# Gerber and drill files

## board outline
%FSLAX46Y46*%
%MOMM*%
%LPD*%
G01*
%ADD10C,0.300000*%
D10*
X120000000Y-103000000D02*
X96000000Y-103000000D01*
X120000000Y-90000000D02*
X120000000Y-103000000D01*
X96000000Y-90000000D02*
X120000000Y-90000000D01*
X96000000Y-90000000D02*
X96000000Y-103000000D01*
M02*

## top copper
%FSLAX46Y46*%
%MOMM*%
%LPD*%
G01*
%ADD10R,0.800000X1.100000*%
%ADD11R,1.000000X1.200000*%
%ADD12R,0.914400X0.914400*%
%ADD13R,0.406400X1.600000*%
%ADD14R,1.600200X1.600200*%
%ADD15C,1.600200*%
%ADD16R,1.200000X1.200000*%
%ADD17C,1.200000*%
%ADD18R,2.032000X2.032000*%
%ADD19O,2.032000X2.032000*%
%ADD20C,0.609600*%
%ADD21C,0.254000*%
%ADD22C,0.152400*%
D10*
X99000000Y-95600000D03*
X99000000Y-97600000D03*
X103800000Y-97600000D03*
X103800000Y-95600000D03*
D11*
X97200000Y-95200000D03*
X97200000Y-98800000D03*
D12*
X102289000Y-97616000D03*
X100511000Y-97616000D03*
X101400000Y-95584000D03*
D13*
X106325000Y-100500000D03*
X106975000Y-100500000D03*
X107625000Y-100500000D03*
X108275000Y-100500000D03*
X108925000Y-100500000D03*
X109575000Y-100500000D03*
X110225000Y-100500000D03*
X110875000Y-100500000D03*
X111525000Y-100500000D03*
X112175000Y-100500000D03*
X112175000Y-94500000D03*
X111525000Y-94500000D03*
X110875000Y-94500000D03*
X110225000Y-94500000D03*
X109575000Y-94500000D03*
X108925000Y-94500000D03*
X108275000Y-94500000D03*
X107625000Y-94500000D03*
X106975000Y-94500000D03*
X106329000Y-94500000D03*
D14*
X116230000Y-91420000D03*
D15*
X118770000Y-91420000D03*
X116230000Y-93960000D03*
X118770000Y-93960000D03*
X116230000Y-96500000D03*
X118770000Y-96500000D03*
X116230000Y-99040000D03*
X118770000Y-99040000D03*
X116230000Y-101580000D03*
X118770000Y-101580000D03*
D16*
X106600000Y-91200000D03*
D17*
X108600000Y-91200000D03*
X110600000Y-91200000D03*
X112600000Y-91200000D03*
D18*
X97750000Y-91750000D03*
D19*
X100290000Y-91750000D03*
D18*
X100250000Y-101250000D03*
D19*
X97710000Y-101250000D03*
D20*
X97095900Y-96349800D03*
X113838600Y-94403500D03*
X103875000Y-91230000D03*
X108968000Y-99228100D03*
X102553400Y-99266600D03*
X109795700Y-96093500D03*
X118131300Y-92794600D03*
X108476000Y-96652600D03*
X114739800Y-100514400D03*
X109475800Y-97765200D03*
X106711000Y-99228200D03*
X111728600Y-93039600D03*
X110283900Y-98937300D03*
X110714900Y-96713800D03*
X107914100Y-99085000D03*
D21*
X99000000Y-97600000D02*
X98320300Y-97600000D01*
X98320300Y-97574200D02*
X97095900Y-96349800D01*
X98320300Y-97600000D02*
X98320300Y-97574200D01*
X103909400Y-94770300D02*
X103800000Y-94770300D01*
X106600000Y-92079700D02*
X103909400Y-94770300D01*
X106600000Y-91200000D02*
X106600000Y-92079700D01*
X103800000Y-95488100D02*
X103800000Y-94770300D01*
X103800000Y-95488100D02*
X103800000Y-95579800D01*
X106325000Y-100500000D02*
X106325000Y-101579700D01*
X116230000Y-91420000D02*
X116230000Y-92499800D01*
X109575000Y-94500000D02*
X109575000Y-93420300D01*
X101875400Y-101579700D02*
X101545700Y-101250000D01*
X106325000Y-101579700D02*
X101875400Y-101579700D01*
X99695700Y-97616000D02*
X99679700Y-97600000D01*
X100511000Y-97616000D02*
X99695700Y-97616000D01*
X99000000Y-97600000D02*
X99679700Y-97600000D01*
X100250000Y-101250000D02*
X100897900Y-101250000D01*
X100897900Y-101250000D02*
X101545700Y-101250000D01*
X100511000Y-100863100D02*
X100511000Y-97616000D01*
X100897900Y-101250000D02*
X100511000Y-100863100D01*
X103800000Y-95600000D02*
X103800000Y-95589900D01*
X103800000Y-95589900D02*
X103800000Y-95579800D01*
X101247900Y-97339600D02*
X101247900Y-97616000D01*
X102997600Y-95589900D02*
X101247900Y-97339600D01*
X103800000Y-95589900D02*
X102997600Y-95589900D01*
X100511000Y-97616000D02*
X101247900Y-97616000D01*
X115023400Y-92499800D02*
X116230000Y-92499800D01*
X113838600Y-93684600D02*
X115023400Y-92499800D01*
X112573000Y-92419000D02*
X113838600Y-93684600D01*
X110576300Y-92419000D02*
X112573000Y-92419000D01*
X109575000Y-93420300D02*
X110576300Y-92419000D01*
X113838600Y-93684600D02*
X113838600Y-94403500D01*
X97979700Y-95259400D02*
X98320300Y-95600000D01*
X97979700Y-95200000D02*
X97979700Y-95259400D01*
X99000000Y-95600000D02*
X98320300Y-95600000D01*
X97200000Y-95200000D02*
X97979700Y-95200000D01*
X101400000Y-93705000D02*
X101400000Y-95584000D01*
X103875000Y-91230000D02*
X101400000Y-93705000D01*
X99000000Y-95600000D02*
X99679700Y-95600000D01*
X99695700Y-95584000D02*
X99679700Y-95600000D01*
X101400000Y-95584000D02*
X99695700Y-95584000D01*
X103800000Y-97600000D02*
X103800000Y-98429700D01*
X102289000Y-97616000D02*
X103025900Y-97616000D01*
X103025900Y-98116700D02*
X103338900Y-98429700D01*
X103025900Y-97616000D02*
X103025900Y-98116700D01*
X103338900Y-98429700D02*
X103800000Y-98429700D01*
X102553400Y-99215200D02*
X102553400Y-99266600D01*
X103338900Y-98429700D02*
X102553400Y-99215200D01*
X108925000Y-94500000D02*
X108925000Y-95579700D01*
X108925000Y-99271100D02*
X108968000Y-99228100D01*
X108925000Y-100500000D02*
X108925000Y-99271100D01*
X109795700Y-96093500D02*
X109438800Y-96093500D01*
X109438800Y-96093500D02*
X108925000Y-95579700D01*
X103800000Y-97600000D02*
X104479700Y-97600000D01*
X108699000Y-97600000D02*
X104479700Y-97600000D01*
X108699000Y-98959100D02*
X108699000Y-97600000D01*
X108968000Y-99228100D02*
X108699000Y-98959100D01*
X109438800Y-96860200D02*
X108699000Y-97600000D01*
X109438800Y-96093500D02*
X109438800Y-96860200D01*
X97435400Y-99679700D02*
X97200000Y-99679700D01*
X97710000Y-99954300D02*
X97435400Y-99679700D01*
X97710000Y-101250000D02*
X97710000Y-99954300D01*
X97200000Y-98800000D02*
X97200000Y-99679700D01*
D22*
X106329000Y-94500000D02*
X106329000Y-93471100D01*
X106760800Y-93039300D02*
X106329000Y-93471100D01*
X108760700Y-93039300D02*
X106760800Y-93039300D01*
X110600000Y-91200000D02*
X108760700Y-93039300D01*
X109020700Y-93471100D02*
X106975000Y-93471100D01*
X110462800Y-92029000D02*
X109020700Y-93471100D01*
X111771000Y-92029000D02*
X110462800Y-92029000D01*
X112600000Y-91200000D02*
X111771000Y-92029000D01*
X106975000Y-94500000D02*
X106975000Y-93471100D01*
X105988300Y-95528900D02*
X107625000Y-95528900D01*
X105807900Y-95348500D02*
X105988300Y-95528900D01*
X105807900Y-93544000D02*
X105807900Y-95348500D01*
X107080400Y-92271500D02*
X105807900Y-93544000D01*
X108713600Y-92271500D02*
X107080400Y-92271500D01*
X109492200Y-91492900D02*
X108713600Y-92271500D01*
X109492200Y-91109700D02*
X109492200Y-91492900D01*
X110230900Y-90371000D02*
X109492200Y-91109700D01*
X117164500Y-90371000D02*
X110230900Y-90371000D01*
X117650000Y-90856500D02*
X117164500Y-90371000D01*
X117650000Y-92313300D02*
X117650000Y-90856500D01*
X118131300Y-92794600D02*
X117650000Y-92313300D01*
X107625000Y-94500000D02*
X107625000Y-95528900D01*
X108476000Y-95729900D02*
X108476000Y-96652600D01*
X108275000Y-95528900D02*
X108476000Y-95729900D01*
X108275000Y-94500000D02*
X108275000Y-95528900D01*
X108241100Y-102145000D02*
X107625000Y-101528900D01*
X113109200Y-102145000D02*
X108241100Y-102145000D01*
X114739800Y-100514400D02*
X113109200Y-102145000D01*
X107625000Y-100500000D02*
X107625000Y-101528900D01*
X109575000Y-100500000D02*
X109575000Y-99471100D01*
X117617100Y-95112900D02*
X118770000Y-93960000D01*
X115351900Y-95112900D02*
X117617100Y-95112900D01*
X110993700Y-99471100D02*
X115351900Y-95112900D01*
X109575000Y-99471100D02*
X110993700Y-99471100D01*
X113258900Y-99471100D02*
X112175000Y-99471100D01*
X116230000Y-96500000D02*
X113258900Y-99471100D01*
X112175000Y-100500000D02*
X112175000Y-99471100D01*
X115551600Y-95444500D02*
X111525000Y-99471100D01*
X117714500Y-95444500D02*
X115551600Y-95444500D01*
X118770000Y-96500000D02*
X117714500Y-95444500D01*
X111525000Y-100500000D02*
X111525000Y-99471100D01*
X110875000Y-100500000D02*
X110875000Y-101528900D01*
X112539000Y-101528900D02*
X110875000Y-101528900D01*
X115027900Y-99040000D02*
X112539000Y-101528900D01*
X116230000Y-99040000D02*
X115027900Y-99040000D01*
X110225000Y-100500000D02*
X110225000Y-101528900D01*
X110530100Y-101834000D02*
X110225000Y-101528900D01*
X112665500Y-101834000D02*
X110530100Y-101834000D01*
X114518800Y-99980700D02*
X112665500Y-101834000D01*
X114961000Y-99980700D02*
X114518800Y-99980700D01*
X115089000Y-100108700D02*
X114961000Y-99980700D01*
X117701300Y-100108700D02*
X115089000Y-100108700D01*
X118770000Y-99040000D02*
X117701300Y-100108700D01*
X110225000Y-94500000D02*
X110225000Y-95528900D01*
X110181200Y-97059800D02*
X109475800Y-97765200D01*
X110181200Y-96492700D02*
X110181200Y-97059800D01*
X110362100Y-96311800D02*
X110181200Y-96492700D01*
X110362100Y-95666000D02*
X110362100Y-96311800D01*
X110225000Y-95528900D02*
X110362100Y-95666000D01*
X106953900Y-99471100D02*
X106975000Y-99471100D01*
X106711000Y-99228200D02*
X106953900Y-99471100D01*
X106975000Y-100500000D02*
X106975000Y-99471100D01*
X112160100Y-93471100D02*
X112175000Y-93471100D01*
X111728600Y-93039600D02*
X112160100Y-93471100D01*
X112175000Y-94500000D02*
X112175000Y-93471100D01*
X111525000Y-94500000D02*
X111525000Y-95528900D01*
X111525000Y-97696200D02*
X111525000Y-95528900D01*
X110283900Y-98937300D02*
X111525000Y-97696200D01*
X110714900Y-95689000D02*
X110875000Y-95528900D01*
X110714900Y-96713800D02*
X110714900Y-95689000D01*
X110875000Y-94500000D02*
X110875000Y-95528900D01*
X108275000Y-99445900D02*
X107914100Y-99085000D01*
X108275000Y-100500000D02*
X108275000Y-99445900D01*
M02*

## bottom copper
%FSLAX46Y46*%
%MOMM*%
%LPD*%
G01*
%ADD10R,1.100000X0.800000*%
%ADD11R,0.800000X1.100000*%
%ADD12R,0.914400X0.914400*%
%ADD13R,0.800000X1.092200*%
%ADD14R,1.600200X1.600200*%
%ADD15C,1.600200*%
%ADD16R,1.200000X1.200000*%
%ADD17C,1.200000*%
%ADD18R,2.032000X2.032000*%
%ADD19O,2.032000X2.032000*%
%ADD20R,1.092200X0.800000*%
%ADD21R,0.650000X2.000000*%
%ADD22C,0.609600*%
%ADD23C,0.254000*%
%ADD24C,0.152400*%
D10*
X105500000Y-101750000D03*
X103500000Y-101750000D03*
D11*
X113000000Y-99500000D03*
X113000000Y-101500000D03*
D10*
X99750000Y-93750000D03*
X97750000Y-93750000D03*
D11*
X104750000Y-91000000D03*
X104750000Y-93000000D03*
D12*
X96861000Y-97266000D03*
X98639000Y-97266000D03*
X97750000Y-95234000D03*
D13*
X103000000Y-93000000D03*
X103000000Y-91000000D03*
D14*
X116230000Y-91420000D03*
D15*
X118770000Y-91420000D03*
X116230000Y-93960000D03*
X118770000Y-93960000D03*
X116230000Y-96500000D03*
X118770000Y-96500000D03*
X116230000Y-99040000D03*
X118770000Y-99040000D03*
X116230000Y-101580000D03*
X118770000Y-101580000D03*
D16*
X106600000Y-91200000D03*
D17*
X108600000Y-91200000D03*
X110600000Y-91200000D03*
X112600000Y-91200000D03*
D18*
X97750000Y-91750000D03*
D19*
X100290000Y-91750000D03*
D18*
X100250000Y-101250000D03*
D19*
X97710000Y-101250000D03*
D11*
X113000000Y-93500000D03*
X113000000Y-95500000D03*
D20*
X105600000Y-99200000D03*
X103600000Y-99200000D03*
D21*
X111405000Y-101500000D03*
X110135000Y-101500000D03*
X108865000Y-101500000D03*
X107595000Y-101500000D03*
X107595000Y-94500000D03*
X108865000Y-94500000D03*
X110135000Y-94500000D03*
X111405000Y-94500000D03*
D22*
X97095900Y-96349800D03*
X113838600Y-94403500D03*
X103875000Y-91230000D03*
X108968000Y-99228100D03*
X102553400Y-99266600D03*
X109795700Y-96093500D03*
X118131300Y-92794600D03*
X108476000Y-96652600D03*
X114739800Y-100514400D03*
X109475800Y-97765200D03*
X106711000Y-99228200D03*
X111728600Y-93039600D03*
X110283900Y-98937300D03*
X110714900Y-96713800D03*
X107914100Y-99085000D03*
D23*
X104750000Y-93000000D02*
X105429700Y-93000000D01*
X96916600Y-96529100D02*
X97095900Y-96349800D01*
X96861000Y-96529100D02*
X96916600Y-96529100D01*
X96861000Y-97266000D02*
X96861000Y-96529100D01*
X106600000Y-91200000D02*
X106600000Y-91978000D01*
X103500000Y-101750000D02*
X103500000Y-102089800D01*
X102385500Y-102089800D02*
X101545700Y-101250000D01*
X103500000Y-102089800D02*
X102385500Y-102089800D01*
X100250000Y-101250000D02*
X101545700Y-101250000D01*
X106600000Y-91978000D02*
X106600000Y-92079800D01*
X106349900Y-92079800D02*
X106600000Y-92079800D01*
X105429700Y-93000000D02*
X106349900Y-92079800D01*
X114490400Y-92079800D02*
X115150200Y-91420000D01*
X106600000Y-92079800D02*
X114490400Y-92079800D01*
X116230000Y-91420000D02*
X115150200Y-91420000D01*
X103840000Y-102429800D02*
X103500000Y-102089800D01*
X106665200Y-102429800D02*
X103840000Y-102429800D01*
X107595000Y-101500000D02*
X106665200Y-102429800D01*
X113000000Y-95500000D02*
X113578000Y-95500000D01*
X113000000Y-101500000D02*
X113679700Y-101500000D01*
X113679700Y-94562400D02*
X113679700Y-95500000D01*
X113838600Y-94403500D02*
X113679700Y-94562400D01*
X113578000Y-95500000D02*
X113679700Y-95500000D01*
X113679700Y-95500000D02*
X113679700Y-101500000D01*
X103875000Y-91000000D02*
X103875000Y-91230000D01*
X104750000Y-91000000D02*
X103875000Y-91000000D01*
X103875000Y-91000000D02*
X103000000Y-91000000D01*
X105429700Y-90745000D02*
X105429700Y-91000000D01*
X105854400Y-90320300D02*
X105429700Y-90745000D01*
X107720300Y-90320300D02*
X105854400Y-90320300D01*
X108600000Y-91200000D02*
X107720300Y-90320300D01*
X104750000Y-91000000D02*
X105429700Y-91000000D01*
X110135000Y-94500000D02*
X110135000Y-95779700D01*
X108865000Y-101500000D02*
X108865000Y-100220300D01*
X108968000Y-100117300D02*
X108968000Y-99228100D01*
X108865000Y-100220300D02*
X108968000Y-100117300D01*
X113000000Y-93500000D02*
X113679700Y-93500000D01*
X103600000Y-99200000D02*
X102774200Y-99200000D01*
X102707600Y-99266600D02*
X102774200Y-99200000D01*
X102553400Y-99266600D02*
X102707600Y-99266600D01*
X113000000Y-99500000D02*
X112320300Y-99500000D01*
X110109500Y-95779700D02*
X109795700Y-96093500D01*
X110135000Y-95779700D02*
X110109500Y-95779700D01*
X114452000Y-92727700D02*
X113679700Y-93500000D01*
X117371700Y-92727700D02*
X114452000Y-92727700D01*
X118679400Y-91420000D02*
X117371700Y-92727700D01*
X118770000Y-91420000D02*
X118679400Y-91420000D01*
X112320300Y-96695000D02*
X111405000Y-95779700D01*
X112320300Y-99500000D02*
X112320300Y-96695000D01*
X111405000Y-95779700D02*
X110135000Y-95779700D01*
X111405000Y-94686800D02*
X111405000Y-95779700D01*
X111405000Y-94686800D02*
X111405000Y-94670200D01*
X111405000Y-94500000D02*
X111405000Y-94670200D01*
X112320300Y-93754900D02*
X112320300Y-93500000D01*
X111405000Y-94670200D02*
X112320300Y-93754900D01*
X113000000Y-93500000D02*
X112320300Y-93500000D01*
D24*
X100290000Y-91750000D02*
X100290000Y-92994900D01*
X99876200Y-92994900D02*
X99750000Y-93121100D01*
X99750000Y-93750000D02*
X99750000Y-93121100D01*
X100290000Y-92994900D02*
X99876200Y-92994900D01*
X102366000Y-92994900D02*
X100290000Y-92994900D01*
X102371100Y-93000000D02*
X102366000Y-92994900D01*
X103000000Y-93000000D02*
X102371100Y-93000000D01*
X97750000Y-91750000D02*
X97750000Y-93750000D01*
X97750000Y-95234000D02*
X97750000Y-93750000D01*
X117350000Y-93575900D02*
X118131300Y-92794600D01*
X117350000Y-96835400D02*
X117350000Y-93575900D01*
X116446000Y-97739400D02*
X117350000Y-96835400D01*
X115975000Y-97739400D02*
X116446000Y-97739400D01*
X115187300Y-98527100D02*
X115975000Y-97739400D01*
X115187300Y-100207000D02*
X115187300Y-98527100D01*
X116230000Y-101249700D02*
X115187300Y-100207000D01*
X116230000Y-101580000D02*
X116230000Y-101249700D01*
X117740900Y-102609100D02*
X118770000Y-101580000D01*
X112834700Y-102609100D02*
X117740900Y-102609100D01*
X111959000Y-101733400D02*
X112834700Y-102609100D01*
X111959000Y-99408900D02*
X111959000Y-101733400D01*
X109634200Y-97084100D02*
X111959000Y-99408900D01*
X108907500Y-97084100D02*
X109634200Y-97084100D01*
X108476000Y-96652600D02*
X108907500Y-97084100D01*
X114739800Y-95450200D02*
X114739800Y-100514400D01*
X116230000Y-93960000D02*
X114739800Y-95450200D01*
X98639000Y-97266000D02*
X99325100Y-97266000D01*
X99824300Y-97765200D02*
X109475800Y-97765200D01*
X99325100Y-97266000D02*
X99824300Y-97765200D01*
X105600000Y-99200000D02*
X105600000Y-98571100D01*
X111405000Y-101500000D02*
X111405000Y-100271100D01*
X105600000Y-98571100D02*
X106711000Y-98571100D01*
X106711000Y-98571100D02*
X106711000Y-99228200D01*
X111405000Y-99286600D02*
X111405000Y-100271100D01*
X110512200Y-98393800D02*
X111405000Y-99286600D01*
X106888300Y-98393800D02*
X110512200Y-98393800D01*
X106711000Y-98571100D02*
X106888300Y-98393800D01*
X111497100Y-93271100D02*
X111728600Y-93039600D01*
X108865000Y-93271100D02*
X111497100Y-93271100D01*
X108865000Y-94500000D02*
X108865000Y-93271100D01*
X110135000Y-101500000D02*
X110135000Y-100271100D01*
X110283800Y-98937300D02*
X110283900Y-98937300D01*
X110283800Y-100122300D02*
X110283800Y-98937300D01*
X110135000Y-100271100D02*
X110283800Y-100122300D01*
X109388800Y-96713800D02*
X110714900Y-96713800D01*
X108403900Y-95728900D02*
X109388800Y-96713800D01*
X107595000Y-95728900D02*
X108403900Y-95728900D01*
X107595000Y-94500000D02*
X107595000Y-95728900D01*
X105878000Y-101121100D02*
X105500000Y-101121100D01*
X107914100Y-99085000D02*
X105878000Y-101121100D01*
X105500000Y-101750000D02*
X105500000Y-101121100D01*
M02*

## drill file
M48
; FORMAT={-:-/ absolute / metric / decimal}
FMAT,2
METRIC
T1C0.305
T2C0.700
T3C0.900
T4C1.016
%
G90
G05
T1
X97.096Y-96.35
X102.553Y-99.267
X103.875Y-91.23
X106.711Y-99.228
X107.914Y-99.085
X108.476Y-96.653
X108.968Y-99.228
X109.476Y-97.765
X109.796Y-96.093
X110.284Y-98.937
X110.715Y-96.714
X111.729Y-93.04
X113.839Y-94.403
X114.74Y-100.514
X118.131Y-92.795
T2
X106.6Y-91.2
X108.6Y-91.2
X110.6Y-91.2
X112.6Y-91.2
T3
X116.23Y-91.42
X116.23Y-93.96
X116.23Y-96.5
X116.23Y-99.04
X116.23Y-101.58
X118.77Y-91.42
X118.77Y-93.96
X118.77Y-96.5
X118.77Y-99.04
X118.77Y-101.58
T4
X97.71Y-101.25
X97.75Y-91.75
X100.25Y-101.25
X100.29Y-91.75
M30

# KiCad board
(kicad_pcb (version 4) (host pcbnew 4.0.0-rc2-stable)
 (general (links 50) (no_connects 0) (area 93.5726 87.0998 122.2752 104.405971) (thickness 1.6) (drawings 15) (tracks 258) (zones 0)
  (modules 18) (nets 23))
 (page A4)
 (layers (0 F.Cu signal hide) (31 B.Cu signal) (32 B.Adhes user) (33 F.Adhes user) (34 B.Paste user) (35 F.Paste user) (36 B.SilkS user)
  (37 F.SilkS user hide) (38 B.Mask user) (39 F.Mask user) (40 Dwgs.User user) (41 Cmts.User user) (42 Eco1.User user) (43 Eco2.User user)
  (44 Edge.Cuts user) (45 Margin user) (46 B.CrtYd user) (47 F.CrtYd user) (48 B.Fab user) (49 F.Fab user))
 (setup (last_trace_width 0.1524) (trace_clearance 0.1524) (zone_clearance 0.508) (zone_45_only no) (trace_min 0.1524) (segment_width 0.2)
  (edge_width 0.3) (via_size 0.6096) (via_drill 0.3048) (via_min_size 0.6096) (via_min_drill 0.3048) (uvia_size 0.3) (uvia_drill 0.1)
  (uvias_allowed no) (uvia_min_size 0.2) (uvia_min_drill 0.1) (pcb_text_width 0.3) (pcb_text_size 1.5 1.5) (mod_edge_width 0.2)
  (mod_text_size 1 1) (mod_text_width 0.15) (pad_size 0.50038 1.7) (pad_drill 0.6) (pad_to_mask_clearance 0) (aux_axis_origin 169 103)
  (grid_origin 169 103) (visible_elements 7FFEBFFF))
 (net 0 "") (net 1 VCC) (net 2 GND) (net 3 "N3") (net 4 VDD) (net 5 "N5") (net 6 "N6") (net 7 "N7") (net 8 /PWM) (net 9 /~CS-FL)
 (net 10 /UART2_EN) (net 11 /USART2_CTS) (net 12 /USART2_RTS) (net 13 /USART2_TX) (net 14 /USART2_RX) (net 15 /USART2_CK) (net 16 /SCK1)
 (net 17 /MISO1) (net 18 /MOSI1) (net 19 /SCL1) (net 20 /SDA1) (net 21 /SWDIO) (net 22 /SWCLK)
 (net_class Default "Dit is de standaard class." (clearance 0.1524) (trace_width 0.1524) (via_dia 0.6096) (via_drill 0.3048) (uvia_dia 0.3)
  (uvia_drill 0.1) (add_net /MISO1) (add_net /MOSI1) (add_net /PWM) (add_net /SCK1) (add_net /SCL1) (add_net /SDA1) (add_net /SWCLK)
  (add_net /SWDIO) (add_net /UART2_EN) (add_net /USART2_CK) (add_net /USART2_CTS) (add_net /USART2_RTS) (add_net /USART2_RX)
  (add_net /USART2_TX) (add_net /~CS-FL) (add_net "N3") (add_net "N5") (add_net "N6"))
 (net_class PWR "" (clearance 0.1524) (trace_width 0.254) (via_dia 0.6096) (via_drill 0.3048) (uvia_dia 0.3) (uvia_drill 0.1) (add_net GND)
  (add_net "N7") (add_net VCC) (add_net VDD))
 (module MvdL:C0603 (layer F.Cu) (at 99 96.6 270)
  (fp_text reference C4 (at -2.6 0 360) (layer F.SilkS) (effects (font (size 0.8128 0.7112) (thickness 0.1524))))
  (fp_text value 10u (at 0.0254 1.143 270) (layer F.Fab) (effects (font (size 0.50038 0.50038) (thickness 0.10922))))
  (pad 1 smd rect (at -1 0 270) (size 1.1 0.8) (layers F.Cu F.Paste F.Mask) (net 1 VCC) (clearance 0.1524))
  (pad 2 smd rect (at 1 0 270) (size 1.1 0.8) (layers F.Cu F.Paste F.Mask) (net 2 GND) (clearance 0.1524)))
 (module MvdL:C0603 (layer B.Cu) (at 104.5 101.75 180)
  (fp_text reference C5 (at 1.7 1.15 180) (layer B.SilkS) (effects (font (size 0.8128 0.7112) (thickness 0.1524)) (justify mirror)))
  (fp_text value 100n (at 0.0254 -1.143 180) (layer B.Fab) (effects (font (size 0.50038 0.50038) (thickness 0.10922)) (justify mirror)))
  (pad 1 smd rect (at -1 0 180) (size 1.1 0.8) (layers B.Cu B.Paste B.Mask) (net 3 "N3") (clearance 0.1524))
  (pad 2 smd rect (at 1 0 180) (size 1.1 0.8) (layers B.Cu B.Paste B.Mask) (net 2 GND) (clearance 0.1524)))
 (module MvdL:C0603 (layer F.Cu) (at 103.8 96.6 90)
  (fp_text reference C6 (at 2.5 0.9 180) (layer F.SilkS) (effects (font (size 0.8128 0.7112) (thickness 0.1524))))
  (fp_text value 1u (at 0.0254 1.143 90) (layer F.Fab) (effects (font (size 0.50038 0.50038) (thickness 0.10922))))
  (pad 1 smd rect (at -1 0 90) (size 1.1 0.8) (layers F.Cu F.Paste F.Mask) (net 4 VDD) (clearance 0.1524))
  (pad 2 smd rect (at 1 0 90) (size 1.1 0.8) (layers F.Cu F.Paste F.Mask) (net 2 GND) (clearance 0.1524)))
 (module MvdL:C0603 (layer B.Cu) (at 113 100.5 270)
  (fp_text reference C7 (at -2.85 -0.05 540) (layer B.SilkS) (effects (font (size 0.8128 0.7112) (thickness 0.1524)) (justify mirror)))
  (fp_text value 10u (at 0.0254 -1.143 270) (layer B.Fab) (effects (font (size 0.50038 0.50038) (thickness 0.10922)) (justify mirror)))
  (pad 1 smd rect (at -1 0 270) (size 1.1 0.8) (layers B.Cu B.Paste B.Mask) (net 4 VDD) (clearance 0.1524))
  (pad 2 smd rect (at 1 0 270) (size 1.1 0.8) (layers B.Cu B.Paste B.Mask) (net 2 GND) (clearance 0.1524)))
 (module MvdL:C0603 (layer B.Cu) (at 98.75 93.75 180)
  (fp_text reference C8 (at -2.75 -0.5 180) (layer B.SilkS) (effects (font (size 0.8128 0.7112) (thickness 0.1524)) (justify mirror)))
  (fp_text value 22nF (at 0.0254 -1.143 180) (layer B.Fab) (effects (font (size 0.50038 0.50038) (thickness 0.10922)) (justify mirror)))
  (pad 1 smd rect (at -1 0 180) (size 1.1 0.8) (layers B.Cu B.Paste B.Mask) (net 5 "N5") (clearance 0.1524))
  (pad 2 smd rect (at 1 0 180) (size 1.1 0.8) (layers B.Cu B.Paste B.Mask) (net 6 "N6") (clearance 0.1524)))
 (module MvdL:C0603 (layer B.Cu) (at 104.75 92 270)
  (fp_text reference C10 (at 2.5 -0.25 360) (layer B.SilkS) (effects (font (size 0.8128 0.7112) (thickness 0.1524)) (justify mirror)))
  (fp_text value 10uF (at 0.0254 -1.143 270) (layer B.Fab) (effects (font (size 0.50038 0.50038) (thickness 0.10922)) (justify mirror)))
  (pad 1 smd rect (at -1 0 270) (size 1.1 0.8) (layers B.Cu B.Paste B.Mask) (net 1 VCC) (clearance 0.1524))
  (pad 2 smd rect (at 1 0 270) (size 1.1 0.8) (layers B.Cu B.Paste B.Mask) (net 2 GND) (clearance 0.1524)))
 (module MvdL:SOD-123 (layer F.Cu) (at 97.2 97 270)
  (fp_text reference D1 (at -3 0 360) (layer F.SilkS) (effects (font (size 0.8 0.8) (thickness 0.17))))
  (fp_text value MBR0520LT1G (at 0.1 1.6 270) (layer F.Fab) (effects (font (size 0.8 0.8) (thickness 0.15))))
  (pad C smd rect (at -1.8 0 270) (size 1.2 1) (layers F.Cu F.Paste F.Mask) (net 1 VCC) (clearance 0.1524))
  (pad A smd rect (at 1.8 0 270) (size 1.2 1) (layers F.Cu F.Paste F.Mask) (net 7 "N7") (clearance 0.1524)))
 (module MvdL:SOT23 (layer B.Cu) (at 97.75 96.25)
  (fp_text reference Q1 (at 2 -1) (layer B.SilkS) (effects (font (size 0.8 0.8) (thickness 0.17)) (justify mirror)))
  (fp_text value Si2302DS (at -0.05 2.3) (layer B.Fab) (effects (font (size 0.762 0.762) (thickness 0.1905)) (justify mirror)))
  (pad 2 smd rect (at -0.889 1.016) (size 0.9144 0.9144) (layers B.Cu B.Paste B.Mask) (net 2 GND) (die_length -2147.483648)
   (clearance 0.1524))
  (pad 1 smd rect (at 0.889 1.016) (size 0.9144 0.9144) (layers B.Cu B.Paste B.Mask) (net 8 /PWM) (clearance 0.1524))
  (pad 3 smd rect (at 0 -1.016) (size 0.9144 0.9144) (layers B.Cu B.Paste B.Mask) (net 6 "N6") (clearance 0.1524)))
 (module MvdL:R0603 (layer B.Cu) (at 103 92 90)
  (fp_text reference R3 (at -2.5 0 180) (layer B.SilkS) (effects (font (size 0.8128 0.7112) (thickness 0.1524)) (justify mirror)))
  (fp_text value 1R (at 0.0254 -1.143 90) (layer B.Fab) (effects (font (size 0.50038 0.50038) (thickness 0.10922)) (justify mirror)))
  (pad 1 smd rect (at -1 0 90) (size 1.0922 0.8) (layers B.Cu B.Paste B.Mask) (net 5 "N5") (clearance 0.1524))
  (pad 2 smd rect (at 1 0 90) (size 1.0922 0.8) (layers B.Cu B.Paste B.Mask) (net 1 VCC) (clearance 0.1524)))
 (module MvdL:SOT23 (layer F.Cu) (at 101.4 96.6 180)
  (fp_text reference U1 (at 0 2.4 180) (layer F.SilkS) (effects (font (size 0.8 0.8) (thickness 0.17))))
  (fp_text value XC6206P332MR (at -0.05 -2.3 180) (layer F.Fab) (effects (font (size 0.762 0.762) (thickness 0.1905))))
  (pad 2 smd rect (at -0.889 -1.016 180) (size 0.9144 0.9144) (layers F.Cu F.Paste F.Mask) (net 4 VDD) (die_length -2147.483648)
   (clearance 0.1524))
  (pad 1 smd rect (at 0.889 -1.016 180) (size 0.9144 0.9144) (layers F.Cu F.Paste F.Mask) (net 2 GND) (clearance 0.1524))
  (pad 3 smd rect (at 0 1.016 180) (size 0.9144 0.9144) (layers F.Cu F.Paste F.Mask) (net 1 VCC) (clearance 0.1524)))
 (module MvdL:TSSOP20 (layer F.Cu) (at 109.25 97.5)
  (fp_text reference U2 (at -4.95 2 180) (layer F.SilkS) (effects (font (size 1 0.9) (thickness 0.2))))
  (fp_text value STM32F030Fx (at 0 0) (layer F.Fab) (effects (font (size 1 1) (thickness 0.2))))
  (pad 1 smd rect (at -2.925 3) (size 0.4064 1.6) (layers F.Cu F.Paste F.Mask) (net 2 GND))
  (pad 2 smd rect (at -2.275 3) (size 0.4064 1.6) (layers F.Cu F.Paste F.Mask) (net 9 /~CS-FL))
  (pad 3 smd rect (at -1.625 3) (size 0.4064 1.6) (layers F.Cu F.Paste F.Mask) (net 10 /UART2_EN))
  (pad 4 smd rect (at -0.975 3) (size 0.4064 1.6) (layers F.Cu F.Paste F.Mask) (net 3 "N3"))
  (pad 5 smd rect (at -0.325 3) (size 0.4064 1.6) (layers F.Cu F.Paste F.Mask) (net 4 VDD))
  (pad 6 smd rect (at 0.325 3) (size 0.4064 1.6) (layers F.Cu F.Paste F.Mask) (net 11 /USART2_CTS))
  (pad 7 smd rect (at 0.975 3) (size 0.4064 1.6) (layers F.Cu F.Paste F.Mask) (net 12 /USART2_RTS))
  (pad 8 smd rect (at 1.625 3) (size 0.4064 1.6) (layers F.Cu F.Paste F.Mask) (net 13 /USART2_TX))
  (pad 9 smd rect (at 2.275 3) (size 0.4064 1.6) (layers F.Cu F.Paste F.Mask) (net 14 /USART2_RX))
  (pad 10 smd rect (at 2.925 3) (size 0.4064 1.6) (layers F.Cu F.Paste F.Mask) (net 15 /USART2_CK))
  (pad 11 smd rect (at 2.925 -3) (size 0.4064 1.6) (layers F.Cu F.Paste F.Mask) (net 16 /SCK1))
  (pad 12 smd rect (at 2.275 -3) (size 0.4064 1.6) (layers F.Cu F.Paste F.Mask) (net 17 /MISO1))
  (pad 13 smd rect (at 1.625 -3) (size 0.4064 1.6) (layers F.Cu F.Paste F.Mask) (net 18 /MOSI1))
  (pad 14 smd rect (at 0.975 -3) (size 0.4064 1.6) (layers F.Cu F.Paste F.Mask) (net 8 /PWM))
  (pad 15 smd rect (at 0.325 -3) (size 0.4064 1.6) (layers F.Cu F.Paste F.Mask) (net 2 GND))
  (pad 16 smd rect (at -0.325 -3) (size 0.4064 1.6) (layers F.Cu F.Paste F.Mask) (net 4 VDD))
  (pad 17 smd rect (at -0.975 -3) (size 0.4064 1.6) (layers F.Cu F.Paste F.Mask) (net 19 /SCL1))
  (pad 18 smd rect (at -1.625 -3) (size 0.4064 1.6) (layers F.Cu F.Paste F.Mask) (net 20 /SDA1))
  (pad 19 smd rect (at -2.275 -3) (size 0.4064 1.6) (layers F.Cu F.Paste F.Mask) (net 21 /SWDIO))
  (pad 20 smd rect (at -2.921 -3) (size 0.4064 1.6) (layers F.Cu F.Paste F.Mask) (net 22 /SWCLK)))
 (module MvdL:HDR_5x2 (layer F.Cu) (at 117.5 96.5 270)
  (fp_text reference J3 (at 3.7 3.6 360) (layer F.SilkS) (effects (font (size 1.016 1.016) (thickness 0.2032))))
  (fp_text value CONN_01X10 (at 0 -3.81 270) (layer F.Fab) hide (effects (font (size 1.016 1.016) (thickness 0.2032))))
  (pad 1 thru_hole rect (at -5.08 1.27 270) (size 1.6002 1.6002) (drill 0.9) (layers *.Cu *.Mask F.SilkS) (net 2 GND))
  (pad 2 thru_hole circle (at -5.08 -1.27 270) (size 1.6002 1.6002) (drill 0.9) (layers *.Cu *.Mask F.SilkS) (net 4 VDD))
  (pad 3 thru_hole circle (at -2.54 1.27 270) (size 1.6002 1.6002) (drill 0.9) (layers *.Cu *.Mask F.SilkS) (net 10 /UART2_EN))
  (pad 4 thru_hole circle (at -2.54 -1.27 270) (size 1.6002 1.6002) (drill 0.9) (layers *.Cu *.Mask F.SilkS) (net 11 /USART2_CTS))
  (pad 5 thru_hole circle (at 0 1.27 270) (size 1.6002 1.6002) (drill 0.9) (layers *.Cu *.Mask F.SilkS) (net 15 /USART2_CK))
  (pad 6 thru_hole circle (at 0 -1.27 270) (size 1.6002 1.6002) (drill 0.9) (layers *.Cu *.Mask F.SilkS) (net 14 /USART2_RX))
  (pad 7 thru_hole circle (at 2.54 1.27 270) (size 1.6002 1.6002) (drill 0.9) (layers *.Cu *.Mask F.SilkS) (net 13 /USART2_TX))
  (pad 8 thru_hole circle (at 2.54 -1.27 270) (size 1.6002 1.6002) (drill 0.9) (layers *.Cu *.Mask F.SilkS) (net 12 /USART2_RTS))
  (pad 9 thru_hole circle (at 5.08 1.27 270) (size 1.6002 1.6002) (drill 0.9) (layers *.Cu *.Mask F.SilkS) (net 20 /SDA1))
  (pad 10 thru_hole circle (at 5.08 -1.27 270) (size 1.6002 1.6002) (drill 0.9) (layers *.Cu *.Mask F.SilkS) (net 19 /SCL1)))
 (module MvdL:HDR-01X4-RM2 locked (layer F.Cu) (at 106.6 91.2)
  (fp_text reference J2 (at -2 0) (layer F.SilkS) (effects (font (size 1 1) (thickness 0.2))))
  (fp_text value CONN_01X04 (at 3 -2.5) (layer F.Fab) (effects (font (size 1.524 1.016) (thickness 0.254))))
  (pad 1 thru_hole rect (at 0 0) (size 1.2 1.2) (drill 0.7) (layers *.Cu *.Mask F.SilkS) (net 2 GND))
  (pad 2 thru_hole circle (at 2 0) (size 1.2 1.2) (drill 0.7) (layers *.Cu *.Mask F.SilkS) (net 1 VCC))
  (pad 3 thru_hole circle (at 4 0) (size 1.2 1.2) (drill 0.7) (layers *.Cu *.Mask F.SilkS) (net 22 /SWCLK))
  (pad 4 thru_hole circle (at 6 0) (size 1.2 1.2) (drill 0.7) (layers *.Cu *.Mask F.SilkS) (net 21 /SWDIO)))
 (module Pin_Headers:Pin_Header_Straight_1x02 (layer F.Cu) (at 97.75 91.75 90)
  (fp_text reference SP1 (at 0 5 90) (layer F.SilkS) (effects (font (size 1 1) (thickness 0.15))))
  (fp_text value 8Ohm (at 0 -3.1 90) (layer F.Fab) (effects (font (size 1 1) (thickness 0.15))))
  (pad 1 thru_hole rect (at 0 0 90) (size 2.032 2.032) (drill 1.016) (layers *.Cu *.Mask F.SilkS) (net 6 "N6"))
  (pad 2 thru_hole oval (at 0 2.54 90) (size 2.032 2.032) (drill 1.016) (layers *.Cu *.Mask F.SilkS) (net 5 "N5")))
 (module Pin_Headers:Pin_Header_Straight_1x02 (layer F.Cu) (at 100.25 101.25 270)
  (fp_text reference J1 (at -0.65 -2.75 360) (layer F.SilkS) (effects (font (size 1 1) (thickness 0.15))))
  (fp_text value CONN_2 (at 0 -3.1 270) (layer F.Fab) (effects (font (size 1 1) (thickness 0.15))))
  (pad 1 thru_hole rect (at 0 0 270) (size 2.032 2.032) (drill 1.016) (layers *.Cu *.Mask F.SilkS) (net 2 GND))
  (pad 2 thru_hole oval (at 0 2.54 270) (size 2.032 2.032) (drill 1.016) (layers *.Cu *.Mask F.SilkS) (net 7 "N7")))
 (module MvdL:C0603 (layer B.Cu) (at 113 94.5 270)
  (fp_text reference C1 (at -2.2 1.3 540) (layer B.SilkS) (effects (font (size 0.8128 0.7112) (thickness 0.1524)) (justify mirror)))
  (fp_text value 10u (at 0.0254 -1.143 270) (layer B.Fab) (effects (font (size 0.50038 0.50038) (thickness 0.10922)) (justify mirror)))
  (pad 1 smd rect (at -1 0 270) (size 1.1 0.8) (layers B.Cu B.Paste B.Mask) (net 4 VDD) (clearance 0.1524))
  (pad 2 smd rect (at 1 0 270) (size 1.1 0.8) (layers B.Cu B.Paste B.Mask) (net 2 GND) (clearance 0.1524)))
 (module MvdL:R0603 (layer B.Cu) (at 104.6 99.2 180)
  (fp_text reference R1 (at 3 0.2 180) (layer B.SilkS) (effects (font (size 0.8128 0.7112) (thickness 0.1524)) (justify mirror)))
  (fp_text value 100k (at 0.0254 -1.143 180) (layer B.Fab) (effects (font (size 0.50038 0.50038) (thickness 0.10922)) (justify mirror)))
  (pad 1 smd rect (at -1 0 180) (size 1.0922 0.8) (layers B.Cu B.Paste B.Mask) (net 9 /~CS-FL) (clearance 0.1524))
  (pad 2 smd rect (at 1 0 180) (size 1.0922 0.8) (layers B.Cu B.Paste B.Mask) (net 4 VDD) (clearance 0.1524)))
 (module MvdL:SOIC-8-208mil (layer B.Cu) (at 109.5 98 90)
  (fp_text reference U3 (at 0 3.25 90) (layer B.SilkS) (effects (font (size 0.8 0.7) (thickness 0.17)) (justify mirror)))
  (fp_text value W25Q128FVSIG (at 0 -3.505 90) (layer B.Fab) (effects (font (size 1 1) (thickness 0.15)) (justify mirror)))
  (pad 1 smd rect (at -3.5 1.905 90) (size 2 0.65) (layers B.Cu B.Paste B.Mask) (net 9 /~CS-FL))
  (pad 2 smd rect (at -3.5 0.635 90) (size 2 0.65) (layers B.Cu B.Paste B.Mask) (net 17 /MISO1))
  (pad 3 smd rect (at -3.5 -0.635 90) (size 2 0.65) (layers B.Cu B.Paste B.Mask) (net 4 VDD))
  (pad 4 smd rect (at -3.5 -1.905 90) (size 2 0.65) (layers B.Cu B.Paste B.Mask) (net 2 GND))
  (pad 5 smd rect (at 3.5 -1.905 90) (size 2 0.65) (layers B.Cu B.Paste B.Mask) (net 18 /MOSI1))
  (pad 6 smd rect (at 3.5 -0.635 90) (size 2 0.65) (layers B.Cu B.Paste B.Mask) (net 16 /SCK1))
  (pad 7 smd rect (at 3.5 0.635 90) (size 2 0.65) (layers B.Cu B.Paste B.Mask) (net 4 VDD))
  (pad 8 smd rect (at 3.5 1.905 90) (size 2 0.65) (layers B.Cu B.Paste B.Mask) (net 4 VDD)))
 (gr_line (start 120 103) (end 96 103) (angle 90) (layer Edge.Cuts) (width 0.3))
 (gr_line (start 120 90) (end 120 103) (angle 90) (layer Edge.Cuts) (width 0.3))
 (gr_line (start 96 90) (end 120 90) (angle 90) (layer Edge.Cuts) (width 0.3))
 (gr_line (start 96 90) (end 96 103) (angle 90) (layer Edge.Cuts) (width 0.3))
 (via (at 97.0959 96.3498) (size 0.6096) (layers F.Cu B.Cu) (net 2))
 (via (at 113.8386 94.4035) (size 0.6096) (layers F.Cu B.Cu) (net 2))
 (segment (start 104.75 93) (end 105.4297 93) (width 0.254) (layer B.Cu) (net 2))
 (segment (start 99 97.6) (end 98.3203 97.6) (width 0.254) (layer F.Cu) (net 2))
 (segment (start 96.9166 96.5291) (end 97.0959 96.3498) (width 0.254) (layer B.Cu) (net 2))
 (segment (start 96.861 96.5291) (end 96.9166 96.5291) (width 0.254) (layer B.Cu) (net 2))
 (segment (start 98.3203 97.5742) (end 97.0959 96.3498) (width 0.254) (layer F.Cu) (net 2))
 (segment (start 98.3203 97.6) (end 98.3203 97.5742) (width 0.254) (layer F.Cu) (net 2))
 (segment (start 96.861 97.266) (end 96.861 96.5291) (width 0.254) (layer B.Cu) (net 2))
 (segment (start 103.9094 94.7703) (end 103.8 94.7703) (width 0.254) (layer F.Cu) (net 2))
 (segment (start 106.6 92.0797) (end 103.9094 94.7703) (width 0.254) (layer F.Cu) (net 2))
 (segment (start 106.6 91.2) (end 106.6 92.0797) (width 0.254) (layer F.Cu) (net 2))
 (segment (start 103.8 95.4881) (end 103.8 94.7703) (width 0.254) (layer F.Cu) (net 2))
 (segment (start 103.8 95.4881) (end 103.8 95.5798) (width 0.254) (layer F.Cu) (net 2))
 (segment (start 106.325 100.5) (end 106.325 101.5797) (width 0.254) (layer F.Cu) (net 2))
 (segment (start 106.6 91.2) (end 106.6 91.978) (width 0.254) (layer B.Cu) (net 2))
 (segment (start 116.23 91.42) (end 116.23 92.4998) (width 0.254) (layer F.Cu) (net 2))
 (segment (start 103.5 101.75) (end 103.5 102.0898) (width 0.254) (layer B.Cu) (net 2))
 (segment (start 102.3855 102.0898) (end 101.5457 101.25) (width 0.254) (layer B.Cu) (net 2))
 (segment (start 103.5 102.0898) (end 102.3855 102.0898) (width 0.254) (layer B.Cu) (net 2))
 (segment (start 100.25 101.25) (end 101.5457 101.25) (width 0.254) (layer B.Cu) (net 2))
 (segment (start 109.575 94.5) (end 109.575 93.4203) (width 0.254) (layer F.Cu) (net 2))
 (segment (start 106.6 91.978) (end 106.6 92.0798) (width 0.254) (layer B.Cu) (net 2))
 (segment (start 106.3499 92.0798) (end 106.6 92.0798) (width 0.254) (layer B.Cu) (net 2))
 (segment (start 105.4297 93) (end 106.3499 92.0798) (width 0.254) (layer B.Cu) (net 2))
 (segment (start 114.4904 92.0798) (end 115.1502 91.42) (width 0.254) (layer B.Cu) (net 2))
 (segment (start 106.6 92.0798) (end 114.4904 92.0798) (width 0.254) (layer B.Cu) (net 2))
 (segment (start 116.23 91.42) (end 115.1502 91.42) (width 0.254) (layer B.Cu) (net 2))
 (segment (start 103.84 102.4298) (end 103.5 102.0898) (width 0.254) (layer B.Cu) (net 2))
 (segment (start 106.6652 102.4298) (end 103.84 102.4298) (width 0.254) (layer B.Cu) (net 2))
 (segment (start 107.595 101.5) (end 106.6652 102.4298) (width 0.254) (layer B.Cu) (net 2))
 (segment (start 113 95.5) (end 113.578 95.5) (width 0.254) (layer B.Cu) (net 2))
 (segment (start 113 101.5) (end 113.6797 101.5) (width 0.254) (layer B.Cu) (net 2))
 (segment (start 101.8754 101.5797) (end 101.5457 101.25) (width 0.254) (layer F.Cu) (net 2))
 (segment (start 106.325 101.5797) (end 101.8754 101.5797) (width 0.254) (layer F.Cu) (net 2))
 (segment (start 99.6957 97.616) (end 99.6797 97.6) (width 0.254) (layer F.Cu) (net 2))
 (segment (start 100.511 97.616) (end 99.6957 97.616) (width 0.254) (layer F.Cu) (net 2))
 (segment (start 99 97.6) (end 99.6797 97.6) (width 0.254) (layer F.Cu) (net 2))
 (segment (start 100.25 101.25) (end 100.8979 101.25) (width 0.254) (layer F.Cu) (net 2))
 (segment (start 100.8979 101.25) (end 101.5457 101.25) (width 0.254) (layer F.Cu) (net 2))
 (segment (start 100.511 100.8631) (end 100.511 97.616) (width 0.254) (layer F.Cu) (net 2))
 (segment (start 100.8979 101.25) (end 100.511 100.8631) (width 0.254) (layer F.Cu) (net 2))
 (segment (start 103.8 95.6) (end 103.8 95.5899) (width 0.254) (layer F.Cu) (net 2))
 (segment (start 103.8 95.5899) (end 103.8 95.5798) (width 0.254) (layer F.Cu) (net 2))
 (segment (start 101.2479 97.3396) (end 101.2479 97.616) (width 0.254) (layer F.Cu) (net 2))
 (segment (start 102.9976 95.5899) (end 101.2479 97.3396) (width 0.254) (layer F.Cu) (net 2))
 (segment (start 103.8 95.5899) (end 102.9976 95.5899) (width 0.254) (layer F.Cu) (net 2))
 (segment (start 100.511 97.616) (end 101.2479 97.616) (width 0.254) (layer F.Cu) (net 2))
 (segment (start 113.6797 94.5624) (end 113.6797 95.5) (width 0.254) (layer B.Cu) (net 2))
 (segment (start 113.8386 94.4035) (end 113.6797 94.5624) (width 0.254) (layer B.Cu) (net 2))
 (segment (start 113.578 95.5) (end 113.6797 95.5) (width 0.254) (layer B.Cu) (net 2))
 (segment (start 113.6797 95.5) (end 113.6797 101.5) (width 0.254) (layer B.Cu) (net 2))
 (segment (start 115.0234 92.4998) (end 116.23 92.4998) (width 0.254) (layer F.Cu) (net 2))
 (segment (start 113.8386 93.6846) (end 115.0234 92.4998) (width 0.254) (layer F.Cu) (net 2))
 (segment (start 112.573 92.419) (end 113.8386 93.6846) (width 0.254) (layer F.Cu) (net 2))
 (segment (start 110.5763 92.419) (end 112.573 92.419) (width 0.254) (layer F.Cu) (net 2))
 (segment (start 109.575 93.4203) (end 110.5763 92.419) (width 0.254) (layer F.Cu) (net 2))
 (segment (start 113.8386 93.6846) (end 113.8386 94.4035) (width 0.254) (layer F.Cu) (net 2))
 (via (at 103.875 91.23) (size 0.6096) (layers F.Cu B.Cu) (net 1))
 (segment (start 97.9797 95.2594) (end 98.3203 95.6) (width 0.254) (layer F.Cu) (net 1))
 (segment (start 97.9797 95.2) (end 97.9797 95.2594) (width 0.254) (layer F.Cu) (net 1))
 (segment (start 99 95.6) (end 98.3203 95.6) (width 0.254) (layer F.Cu) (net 1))
 (segment (start 97.2 95.2) (end 97.9797 95.2) (width 0.254) (layer F.Cu) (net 1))
 (segment (start 103.875 91) (end 103.875 91.23) (width 0.254) (layer B.Cu) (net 1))
 (segment (start 104.75 91) (end 103.875 91) (width 0.254) (layer B.Cu) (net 1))
 (segment (start 103.875 91) (end 103 91) (width 0.254) (layer B.Cu) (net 1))
 (segment (start 101.4 93.705) (end 101.4 95.584) (width 0.254) (layer F.Cu) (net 1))
 (segment (start 103.875 91.23) (end 101.4 93.705) (width 0.254) (layer F.Cu) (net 1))
 (segment (start 99 95.6) (end 99.6797 95.6) (width 0.254) (layer F.Cu) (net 1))
 (segment (start 99.6957 95.584) (end 99.6797 95.6) (width 0.254) (layer F.Cu) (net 1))
 (segment (start 101.4 95.584) (end 99.6957 95.584) (width 0.254) (layer F.Cu) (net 1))
 (segment (start 105.4297 90.745) (end 105.4297 91) (width 0.254) (layer B.Cu) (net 1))
 (segment (start 105.8544 90.3203) (end 105.4297 90.745) (width 0.254) (layer B.Cu) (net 1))
 (segment (start 107.7203 90.3203) (end 105.8544 90.3203) (width 0.254) (layer B.Cu) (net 1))
 (segment (start 108.6 91.2) (end 107.7203 90.3203) (width 0.254) (layer B.Cu) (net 1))
 (segment (start 104.75 91) (end 105.4297 91) (width 0.254) (layer B.Cu) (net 1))
 (via (at 108.968 99.2281) (size 0.6096) (layers F.Cu B.Cu) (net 4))
 (via (at 102.5534 99.2666) (size 0.6096) (layers F.Cu B.Cu) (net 4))
 (via (at 109.7957 96.0935) (size 0.6096) (layers F.Cu B.Cu) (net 4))
 (segment (start 110.135 94.5) (end 110.135 95.7797) (width 0.254) (layer B.Cu) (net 4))
 (segment (start 108.865 101.5) (end 108.865 100.2203) (width 0.254) (layer B.Cu) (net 4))
 (segment (start 108.968 100.1173) (end 108.968 99.2281) (width 0.254) (layer B.Cu) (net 4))
 (segment (start 108.865 100.2203) (end 108.968 100.1173) (width 0.254) (layer B.Cu) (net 4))
 (segment (start 113 93.5) (end 113.6797 93.5) (width 0.254) (layer B.Cu) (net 4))
 (segment (start 103.8 97.6) (end 103.8 98.4297) (width 0.254) (layer F.Cu) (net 4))
 (segment (start 102.289 97.616) (end 103.0259 97.616) (width 0.254) (layer F.Cu) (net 4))
 (segment (start 103.0259 98.1167) (end 103.3389 98.4297) (width 0.254) (layer F.Cu) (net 4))
 (segment (start 103.0259 97.616) (end 103.0259 98.1167) (width 0.254) (layer F.Cu) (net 4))
 (segment (start 103.3389 98.4297) (end 103.8 98.4297) (width 0.254) (layer F.Cu) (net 4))
 (segment (start 103.6 99.2) (end 102.7742 99.2) (width 0.254) (layer B.Cu) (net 4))
 (segment (start 102.7076 99.2666) (end 102.7742 99.2) (width 0.254) (layer B.Cu) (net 4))
 (segment (start 102.5534 99.2666) (end 102.7076 99.2666) (width 0.254) (layer B.Cu) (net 4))
 (segment (start 102.5534 99.2152) (end 102.5534 99.2666) (width 0.254) (layer F.Cu) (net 4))
 (segment (start 103.3389 98.4297) (end 102.5534 99.2152) (width 0.254) (layer F.Cu) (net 4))
 (segment (start 113 99.5) (end 112.3203 99.5) (width 0.254) (layer B.Cu) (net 4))
 (segment (start 110.1095 95.7797) (end 109.7957 96.0935) (width 0.254) (layer B.Cu) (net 4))
 (segment (start 110.135 95.7797) (end 110.1095 95.7797) (width 0.254) (layer B.Cu) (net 4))
 (segment (start 108.925 94.5) (end 108.925 95.5797) (width 0.254) (layer F.Cu) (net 4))
 (segment (start 108.925 99.2711) (end 108.968 99.2281) (width 0.254) (layer F.Cu) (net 4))
 (segment (start 108.925 100.5) (end 108.925 99.2711) (width 0.254) (layer F.Cu) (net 4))
 (segment (start 109.7957 96.0935) (end 109.4388 96.0935) (width 0.254) (layer F.Cu) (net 4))
 (segment (start 109.4388 96.0935) (end 108.925 95.5797) (width 0.254) (layer F.Cu) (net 4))
 (segment (start 103.8 97.6) (end 104.4797 97.6) (width 0.254) (layer F.Cu) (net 4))
 (segment (start 108.699 97.6) (end 104.4797 97.6) (width 0.254) (layer F.Cu) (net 4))
 (segment (start 108.699 98.9591) (end 108.699 97.6) (width 0.254) (layer F.Cu) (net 4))
 (segment (start 108.968 99.2281) (end 108.699 98.9591) (width 0.254) (layer F.Cu) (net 4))
 (segment (start 114.452 92.7277) (end 113.6797 93.5) (width 0.254) (layer B.Cu) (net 4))
 (segment (start 117.3717 92.7277) (end 114.452 92.7277) (width 0.254) (layer B.Cu) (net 4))
 (segment (start 118.6794 91.42) (end 117.3717 92.7277) (width 0.254) (layer B.Cu) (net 4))
 (segment (start 118.77 91.42) (end 118.6794 91.42) (width 0.254) (layer B.Cu) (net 4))
 (segment (start 109.4388 96.8602) (end 108.699 97.6) (width 0.254) (layer F.Cu) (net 4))
 (segment (start 109.4388 96.0935) (end 109.4388 96.8602) (width 0.254) (layer F.Cu) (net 4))
 (segment (start 112.3203 96.695) (end 111.405 95.7797) (width 0.254) (layer B.Cu) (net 4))
 (segment (start 112.3203 99.5) (end 112.3203 96.695) (width 0.254) (layer B.Cu) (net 4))
 (segment (start 111.405 95.7797) (end 110.135 95.7797) (width 0.254) (layer B.Cu) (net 4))
 (segment (start 111.405 94.6868) (end 111.405 95.7797) (width 0.254) (layer B.Cu) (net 4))
 (segment (start 111.405 94.6868) (end 111.405 94.6702) (width 0.254) (layer B.Cu) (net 4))
 (segment (start 111.405 94.5) (end 111.405 94.6702) (width 0.254) (layer B.Cu) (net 4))
 (segment (start 112.3203 93.7549) (end 112.3203 93.5) (width 0.254) (layer B.Cu) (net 4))
 (segment (start 111.405 94.6702) (end 112.3203 93.7549) (width 0.254) (layer B.Cu) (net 4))
 (segment (start 113 93.5) (end 112.3203 93.5) (width 0.254) (layer B.Cu) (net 4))
 (segment (start 100.29 91.75) (end 100.29 92.9949) (width 0.1524) (layer B.Cu) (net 5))
 (segment (start 99.8762 92.9949) (end 99.75 93.1211) (width 0.1524) (layer B.Cu) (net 5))
 (segment (start 99.75 93.75) (end 99.75 93.1211) (width 0.1524) (layer B.Cu) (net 5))
 (segment (start 100.29 92.9949) (end 99.8762 92.9949) (width 0.1524) (layer B.Cu) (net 5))
 (segment (start 102.366 92.9949) (end 100.29 92.9949) (width 0.1524) (layer B.Cu) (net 5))
 (segment (start 102.3711 93) (end 102.366 92.9949) (width 0.1524) (layer B.Cu) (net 5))
 (segment (start 103 93) (end 102.3711 93) (width 0.1524) (layer B.Cu) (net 5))
 (segment (start 97.75 91.75) (end 97.75 93.75) (width 0.1524) (layer B.Cu) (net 6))
 (segment (start 97.75 95.234) (end 97.75 93.75) (width 0.1524) (layer B.Cu) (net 6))
 (segment (start 97.4354 99.6797) (end 97.2 99.6797) (width 0.254) (layer F.Cu) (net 7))
 (segment (start 97.71 99.9543) (end 97.4354 99.6797) (width 0.254) (layer F.Cu) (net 7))
 (segment (start 97.71 101.25) (end 97.71 99.9543) (width 0.254) (layer F.Cu) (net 7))
 (segment (start 97.2 98.8) (end 97.2 99.6797) (width 0.254) (layer F.Cu) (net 7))
 (segment (start 106.329 94.5) (end 106.329 93.4711) (width 0.1524) (layer F.Cu) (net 22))
 (segment (start 106.7608 93.0393) (end 106.329 93.4711) (width 0.1524) (layer F.Cu) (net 22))
 (segment (start 108.7607 93.0393) (end 106.7608 93.0393) (width 0.1524) (layer F.Cu) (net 22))
 (segment (start 110.6 91.2) (end 108.7607 93.0393) (width 0.1524) (layer F.Cu) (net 22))
 (segment (start 109.0207 93.4711) (end 106.975 93.4711) (width 0.1524) (layer F.Cu) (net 21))
 (segment (start 110.4628 92.029) (end 109.0207 93.4711) (width 0.1524) (layer F.Cu) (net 21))
 (segment (start 111.771 92.029) (end 110.4628 92.029) (width 0.1524) (layer F.Cu) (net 21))
 (segment (start 112.6 91.2) (end 111.771 92.029) (width 0.1524) (layer F.Cu) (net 21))
 (segment (start 106.975 94.5) (end 106.975 93.4711) (width 0.1524) (layer F.Cu) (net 21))
 (via (at 118.1313 92.7946) (size 0.6096) (layers F.Cu B.Cu) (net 20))
 (segment (start 105.9883 95.5289) (end 107.625 95.5289) (width 0.1524) (layer F.Cu) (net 20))
 (segment (start 105.8079 95.3485) (end 105.9883 95.5289) (width 0.1524) (layer F.Cu) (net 20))
 (segment (start 105.8079 93.544) (end 105.8079 95.3485) (width 0.1524) (layer F.Cu) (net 20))
 (segment (start 107.0804 92.2715) (end 105.8079 93.544) (width 0.1524) (layer F.Cu) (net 20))
 (segment (start 108.7136 92.2715) (end 107.0804 92.2715) (width 0.1524) (layer F.Cu) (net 20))
 (segment (start 109.4922 91.4929) (end 108.7136 92.2715) (width 0.1524) (layer F.Cu) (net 20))
 (segment (start 109.4922 91.1097) (end 109.4922 91.4929) (width 0.1524) (layer F.Cu) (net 20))
 (segment (start 110.2309 90.371) (end 109.4922 91.1097) (width 0.1524) (layer F.Cu) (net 20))
 (segment (start 117.1645 90.371) (end 110.2309 90.371) (width 0.1524) (layer F.Cu) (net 20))
 (segment (start 117.65 90.8565) (end 117.1645 90.371) (width 0.1524) (layer F.Cu) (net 20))
 (segment (start 117.65 92.3133) (end 117.65 90.8565) (width 0.1524) (layer F.Cu) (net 20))
 (segment (start 118.1313 92.7946) (end 117.65 92.3133) (width 0.1524) (layer F.Cu) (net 20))
 (segment (start 107.625 94.5) (end 107.625 95.5289) (width 0.1524) (layer F.Cu) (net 20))
 (segment (start 117.35 93.5759) (end 118.1313 92.7946) (width 0.1524) (layer B.Cu) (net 20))
 (segment (start 117.35 96.8354) (end 117.35 93.5759) (width 0.1524) (layer B.Cu) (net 20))
 (segment (start 116.446 97.7394) (end 117.35 96.8354) (width 0.1524) (layer B.Cu) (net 20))
 (segment (start 115.975 97.7394) (end 116.446 97.7394) (width 0.1524) (layer B.Cu) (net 20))
 (segment (start 115.1873 98.5271) (end 115.975 97.7394) (width 0.1524) (layer B.Cu) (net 20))
 (segment (start 115.1873 100.207) (end 115.1873 98.5271) (width 0.1524) (layer B.Cu) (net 20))
 (segment (start 116.23 101.2497) (end 115.1873 100.207) (width 0.1524) (layer B.Cu) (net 20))
 (segment (start 116.23 101.58) (end 116.23 101.2497) (width 0.1524) (layer B.Cu) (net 20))
 (via (at 108.476 96.6526) (size 0.6096) (layers F.Cu B.Cu) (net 19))
 (segment (start 108.476 95.7299) (end 108.476 96.6526) (width 0.1524) (layer F.Cu) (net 19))
 (segment (start 108.275 95.5289) (end 108.476 95.7299) (width 0.1524) (layer F.Cu) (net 19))
 (segment (start 117.7409 102.6091) (end 118.77 101.58) (width 0.1524) (layer B.Cu) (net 19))
 (segment (start 112.8347 102.6091) (end 117.7409 102.6091) (width 0.1524) (layer B.Cu) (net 19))
 (segment (start 111.959 101.7334) (end 112.8347 102.6091) (width 0.1524) (layer B.Cu) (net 19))
 (segment (start 111.959 99.4089) (end 111.959 101.7334) (width 0.1524) (layer B.Cu) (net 19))
 (segment (start 109.6342 97.0841) (end 111.959 99.4089) (width 0.1524) (layer B.Cu) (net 19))
 (segment (start 108.9075 97.0841) (end 109.6342 97.0841) (width 0.1524) (layer B.Cu) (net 19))
 (segment (start 108.476 96.6526) (end 108.9075 97.0841) (width 0.1524) (layer B.Cu) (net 19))
 (segment (start 108.275 94.5) (end 108.275 95.5289) (width 0.1524) (layer F.Cu) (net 19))
 (via (at 114.7398 100.5144) (size 0.6096) (layers F.Cu B.Cu) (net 10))
 (segment (start 114.7398 95.4502) (end 114.7398 100.5144) (width 0.1524) (layer B.Cu) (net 10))
 (segment (start 116.23 93.96) (end 114.7398 95.4502) (width 0.1524) (layer B.Cu) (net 10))
 (segment (start 108.2411 102.145) (end 107.625 101.5289) (width 0.1524) (layer F.Cu) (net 10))
 (segment (start 113.1092 102.145) (end 108.2411 102.145) (width 0.1524) (layer F.Cu) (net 10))
 (segment (start 114.7398 100.5144) (end 113.1092 102.145) (width 0.1524) (layer F.Cu) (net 10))
 (segment (start 107.625 100.5) (end 107.625 101.5289) (width 0.1524) (layer F.Cu) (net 10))
 (segment (start 109.575 100.5) (end 109.575 99.4711) (width 0.1524) (layer F.Cu) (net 11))
 (segment (start 117.6171 95.1129) (end 118.77 93.96) (width 0.1524) (layer F.Cu) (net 11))
 (segment (start 115.3519 95.1129) (end 117.6171 95.1129) (width 0.1524) (layer F.Cu) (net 11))
 (segment (start 110.9937 99.4711) (end 115.3519 95.1129) (width 0.1524) (layer F.Cu) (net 11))
 (segment (start 109.575 99.4711) (end 110.9937 99.4711) (width 0.1524) (layer F.Cu) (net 11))
 (segment (start 113.2589 99.4711) (end 112.175 99.4711) (width 0.1524) (layer F.Cu) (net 15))
 (segment (start 116.23 96.5) (end 113.2589 99.4711) (width 0.1524) (layer F.Cu) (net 15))
 (segment (start 112.175 100.5) (end 112.175 99.4711) (width 0.1524) (layer F.Cu) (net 15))
 (segment (start 115.5516 95.4445) (end 111.525 99.4711) (width 0.1524) (layer F.Cu) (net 14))
 (segment (start 117.7145 95.4445) (end 115.5516 95.4445) (width 0.1524) (layer F.Cu) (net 14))
 (segment (start 118.77 96.5) (end 117.7145 95.4445) (width 0.1524) (layer F.Cu) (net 14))
 (segment (start 111.525 100.5) (end 111.525 99.4711) (width 0.1524) (layer F.Cu) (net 14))
 (segment (start 110.875 100.5) (end 110.875 101.5289) (width 0.1524) (layer F.Cu) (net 13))
 (segment (start 112.539 101.5289) (end 110.875 101.5289) (width 0.1524) (layer F.Cu) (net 13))
 (segment (start 115.0279 99.04) (end 112.539 101.5289) (width 0.1524) (layer F.Cu) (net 13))
 (segment (start 116.23 99.04) (end 115.0279 99.04) (width 0.1524) (layer F.Cu) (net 13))
 (segment (start 110.225 100.5) (end 110.225 101.5289) (width 0.1524) (layer F.Cu) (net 12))
 (segment (start 110.5301 101.834) (end 110.225 101.5289) (width 0.1524) (layer F.Cu) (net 12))
 (segment (start 112.6655 101.834) (end 110.5301 101.834) (width 0.1524) (layer F.Cu) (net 12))
 (segment (start 114.5188 99.9807) (end 112.6655 101.834) (width 0.1524) (layer F.Cu) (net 12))
 (segment (start 114.961 99.9807) (end 114.5188 99.9807) (width 0.1524) (layer F.Cu) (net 12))
 (segment (start 115.089 100.1087) (end 114.961 99.9807) (width 0.1524) (layer F.Cu) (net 12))
 (segment (start 117.7013 100.1087) (end 115.089 100.1087) (width 0.1524) (layer F.Cu) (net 12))
 (segment (start 118.77 99.04) (end 117.7013 100.1087) (width 0.1524) (layer F.Cu) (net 12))
 (via (at 109.4758 97.7652) (size 0.6096) (layers F.Cu B.Cu) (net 8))
 (segment (start 110.225 94.5) (end 110.225 95.5289) (width 0.1524) (layer F.Cu) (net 8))
 (segment (start 98.639 97.266) (end 99.3251 97.266) (width 0.1524) (layer B.Cu) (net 8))
 (segment (start 99.8243 97.7652) (end 109.4758 97.7652) (width 0.1524) (layer B.Cu) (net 8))
 (segment (start 99.3251 97.266) (end 99.8243 97.7652) (width 0.1524) (layer B.Cu) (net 8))
 (segment (start 110.1812 97.0598) (end 109.4758 97.7652) (width 0.1524) (layer F.Cu) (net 8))
 (segment (start 110.1812 96.4927) (end 110.1812 97.0598) (width 0.1524) (layer F.Cu) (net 8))
 (segment (start 110.3621 96.3118) (end 110.1812 96.4927) (width 0.1524) (layer F.Cu) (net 8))
 (segment (start 110.3621 95.666) (end 110.3621 96.3118) (width 0.1524) (layer F.Cu) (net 8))
 (segment (start 110.225 95.5289) (end 110.3621 95.666) (width 0.1524) (layer F.Cu) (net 8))
 (via (at 106.711 99.2282) (size 0.6096) (layers F.Cu B.Cu) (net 9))
 (segment (start 105.6 99.2) (end 105.6 98.5711) (width 0.1524) (layer B.Cu) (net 9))
 (segment (start 111.405 101.5) (end 111.405 100.2711) (width 0.1524) (layer B.Cu) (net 9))
 (segment (start 106.9539 99.4711) (end 106.975 99.4711) (width 0.1524) (layer F.Cu) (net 9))
 (segment (start 106.711 99.2282) (end 106.9539 99.4711) (width 0.1524) (layer F.Cu) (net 9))
 (segment (start 106.975 100.5) (end 106.975 99.4711) (width 0.1524) (layer F.Cu) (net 9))
 (segment (start 105.6 98.5711) (end 106.711 98.5711) (width 0.1524) (layer B.Cu) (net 9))
 (segment (start 106.711 98.5711) (end 106.711 99.2282) (width 0.1524) (layer B.Cu) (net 9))
 (segment (start 111.405 99.2866) (end 111.405 100.2711) (width 0.1524) (layer B.Cu) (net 9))
 (segment (start 110.5122 98.3938) (end 111.405 99.2866) (width 0.1524) (layer B.Cu) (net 9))
 (segment (start 106.8883 98.3938) (end 110.5122 98.3938) (width 0.1524) (layer B.Cu) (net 9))
 (segment (start 106.711 98.5711) (end 106.8883 98.3938) (width 0.1524) (layer B.Cu) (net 9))
 (via (at 111.7286 93.0396) (size 0.6096) (layers F.Cu B.Cu) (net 16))
 (segment (start 111.4971 93.2711) (end 111.7286 93.0396) (width 0.1524) (layer B.Cu) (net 16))
 (segment (start 108.865 93.2711) (end 111.4971 93.2711) (width 0.1524) (layer B.Cu) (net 16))
 (segment (start 112.1601 93.4711) (end 112.175 93.4711) (width 0.1524) (layer F.Cu) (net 16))
 (segment (start 111.7286 93.0396) (end 112.1601 93.4711) (width 0.1524) (layer F.Cu) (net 16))
 (segment (start 112.175 94.5) (end 112.175 93.4711) (width 0.1524) (layer F.Cu) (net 16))
 (segment (start 108.865 94.5) (end 108.865 93.2711) (width 0.1524) (layer B.Cu) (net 16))
 (via (at 110.2839 98.9373) (size 0.6096) (layers F.Cu B.Cu) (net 17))
 (segment (start 110.135 101.5) (end 110.135 100.2711) (width 0.1524) (layer B.Cu) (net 17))
 (segment (start 110.2838 98.9373) (end 110.2839 98.9373) (width 0.1524) (layer B.Cu) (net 17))
 (segment (start 110.2838 100.1223) (end 110.2838 98.9373) (width 0.1524) (layer B.Cu) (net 17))
 (segment (start 110.135 100.2711) (end 110.2838 100.1223) (width 0.1524) (layer B.Cu) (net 17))
 (segment (start 111.525 94.5) (end 111.525 95.5289) (width 0.1524) (layer F.Cu) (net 17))
 (segment (start 111.525 97.6962) (end 111.525 95.5289) (width 0.1524) (layer F.Cu) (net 17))
 (segment (start 110.2839 98.9373) (end 111.525 97.6962) (width 0.1524) (layer F.Cu) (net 17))
 (via (at 110.7149 96.7138) (size 0.6096) (layers F.Cu B.Cu) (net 18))
 (segment (start 109.3888 96.7138) (end 110.7149 96.7138) (width 0.1524) (layer B.Cu) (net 18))
 (segment (start 108.4039 95.7289) (end 109.3888 96.7138) (width 0.1524) (layer B.Cu) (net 18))
 (segment (start 107.595 95.7289) (end 108.4039 95.7289) (width 0.1524) (layer B.Cu) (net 18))
 (segment (start 110.7149 95.689) (end 110.875 95.5289) (width 0.1524) (layer F.Cu) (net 18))
 (segment (start 110.7149 96.7138) (end 110.7149 95.689) (width 0.1524) (layer F.Cu) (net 18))
 (segment (start 110.875 94.5) (end 110.875 95.5289) (width 0.1524) (layer F.Cu) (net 18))
 (segment (start 107.595 94.5) (end 107.595 95.7289) (width 0.1524) (layer B.Cu) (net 18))
 (via (at 107.9141 99.085) (size 0.6096) (layers F.Cu B.Cu) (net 3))
 (segment (start 108.275 99.4459) (end 107.9141 99.085) (width 0.1524) (layer F.Cu) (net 3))
 (segment (start 108.275 100.5) (end 108.275 99.4459) (width 0.1524) (layer F.Cu) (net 3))
 (segment (start 105.878 101.1211) (end 105.5 101.1211) (width 0.1524) (layer B.Cu) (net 3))
 (segment (start 107.9141 99.085) (end 105.878 101.1211) (width 0.1524) (layer B.Cu) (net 3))
 (segment (start 105.5 101.75) (end 105.5 101.1211) (width 0.1524) (layer B.Cu) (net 3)))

